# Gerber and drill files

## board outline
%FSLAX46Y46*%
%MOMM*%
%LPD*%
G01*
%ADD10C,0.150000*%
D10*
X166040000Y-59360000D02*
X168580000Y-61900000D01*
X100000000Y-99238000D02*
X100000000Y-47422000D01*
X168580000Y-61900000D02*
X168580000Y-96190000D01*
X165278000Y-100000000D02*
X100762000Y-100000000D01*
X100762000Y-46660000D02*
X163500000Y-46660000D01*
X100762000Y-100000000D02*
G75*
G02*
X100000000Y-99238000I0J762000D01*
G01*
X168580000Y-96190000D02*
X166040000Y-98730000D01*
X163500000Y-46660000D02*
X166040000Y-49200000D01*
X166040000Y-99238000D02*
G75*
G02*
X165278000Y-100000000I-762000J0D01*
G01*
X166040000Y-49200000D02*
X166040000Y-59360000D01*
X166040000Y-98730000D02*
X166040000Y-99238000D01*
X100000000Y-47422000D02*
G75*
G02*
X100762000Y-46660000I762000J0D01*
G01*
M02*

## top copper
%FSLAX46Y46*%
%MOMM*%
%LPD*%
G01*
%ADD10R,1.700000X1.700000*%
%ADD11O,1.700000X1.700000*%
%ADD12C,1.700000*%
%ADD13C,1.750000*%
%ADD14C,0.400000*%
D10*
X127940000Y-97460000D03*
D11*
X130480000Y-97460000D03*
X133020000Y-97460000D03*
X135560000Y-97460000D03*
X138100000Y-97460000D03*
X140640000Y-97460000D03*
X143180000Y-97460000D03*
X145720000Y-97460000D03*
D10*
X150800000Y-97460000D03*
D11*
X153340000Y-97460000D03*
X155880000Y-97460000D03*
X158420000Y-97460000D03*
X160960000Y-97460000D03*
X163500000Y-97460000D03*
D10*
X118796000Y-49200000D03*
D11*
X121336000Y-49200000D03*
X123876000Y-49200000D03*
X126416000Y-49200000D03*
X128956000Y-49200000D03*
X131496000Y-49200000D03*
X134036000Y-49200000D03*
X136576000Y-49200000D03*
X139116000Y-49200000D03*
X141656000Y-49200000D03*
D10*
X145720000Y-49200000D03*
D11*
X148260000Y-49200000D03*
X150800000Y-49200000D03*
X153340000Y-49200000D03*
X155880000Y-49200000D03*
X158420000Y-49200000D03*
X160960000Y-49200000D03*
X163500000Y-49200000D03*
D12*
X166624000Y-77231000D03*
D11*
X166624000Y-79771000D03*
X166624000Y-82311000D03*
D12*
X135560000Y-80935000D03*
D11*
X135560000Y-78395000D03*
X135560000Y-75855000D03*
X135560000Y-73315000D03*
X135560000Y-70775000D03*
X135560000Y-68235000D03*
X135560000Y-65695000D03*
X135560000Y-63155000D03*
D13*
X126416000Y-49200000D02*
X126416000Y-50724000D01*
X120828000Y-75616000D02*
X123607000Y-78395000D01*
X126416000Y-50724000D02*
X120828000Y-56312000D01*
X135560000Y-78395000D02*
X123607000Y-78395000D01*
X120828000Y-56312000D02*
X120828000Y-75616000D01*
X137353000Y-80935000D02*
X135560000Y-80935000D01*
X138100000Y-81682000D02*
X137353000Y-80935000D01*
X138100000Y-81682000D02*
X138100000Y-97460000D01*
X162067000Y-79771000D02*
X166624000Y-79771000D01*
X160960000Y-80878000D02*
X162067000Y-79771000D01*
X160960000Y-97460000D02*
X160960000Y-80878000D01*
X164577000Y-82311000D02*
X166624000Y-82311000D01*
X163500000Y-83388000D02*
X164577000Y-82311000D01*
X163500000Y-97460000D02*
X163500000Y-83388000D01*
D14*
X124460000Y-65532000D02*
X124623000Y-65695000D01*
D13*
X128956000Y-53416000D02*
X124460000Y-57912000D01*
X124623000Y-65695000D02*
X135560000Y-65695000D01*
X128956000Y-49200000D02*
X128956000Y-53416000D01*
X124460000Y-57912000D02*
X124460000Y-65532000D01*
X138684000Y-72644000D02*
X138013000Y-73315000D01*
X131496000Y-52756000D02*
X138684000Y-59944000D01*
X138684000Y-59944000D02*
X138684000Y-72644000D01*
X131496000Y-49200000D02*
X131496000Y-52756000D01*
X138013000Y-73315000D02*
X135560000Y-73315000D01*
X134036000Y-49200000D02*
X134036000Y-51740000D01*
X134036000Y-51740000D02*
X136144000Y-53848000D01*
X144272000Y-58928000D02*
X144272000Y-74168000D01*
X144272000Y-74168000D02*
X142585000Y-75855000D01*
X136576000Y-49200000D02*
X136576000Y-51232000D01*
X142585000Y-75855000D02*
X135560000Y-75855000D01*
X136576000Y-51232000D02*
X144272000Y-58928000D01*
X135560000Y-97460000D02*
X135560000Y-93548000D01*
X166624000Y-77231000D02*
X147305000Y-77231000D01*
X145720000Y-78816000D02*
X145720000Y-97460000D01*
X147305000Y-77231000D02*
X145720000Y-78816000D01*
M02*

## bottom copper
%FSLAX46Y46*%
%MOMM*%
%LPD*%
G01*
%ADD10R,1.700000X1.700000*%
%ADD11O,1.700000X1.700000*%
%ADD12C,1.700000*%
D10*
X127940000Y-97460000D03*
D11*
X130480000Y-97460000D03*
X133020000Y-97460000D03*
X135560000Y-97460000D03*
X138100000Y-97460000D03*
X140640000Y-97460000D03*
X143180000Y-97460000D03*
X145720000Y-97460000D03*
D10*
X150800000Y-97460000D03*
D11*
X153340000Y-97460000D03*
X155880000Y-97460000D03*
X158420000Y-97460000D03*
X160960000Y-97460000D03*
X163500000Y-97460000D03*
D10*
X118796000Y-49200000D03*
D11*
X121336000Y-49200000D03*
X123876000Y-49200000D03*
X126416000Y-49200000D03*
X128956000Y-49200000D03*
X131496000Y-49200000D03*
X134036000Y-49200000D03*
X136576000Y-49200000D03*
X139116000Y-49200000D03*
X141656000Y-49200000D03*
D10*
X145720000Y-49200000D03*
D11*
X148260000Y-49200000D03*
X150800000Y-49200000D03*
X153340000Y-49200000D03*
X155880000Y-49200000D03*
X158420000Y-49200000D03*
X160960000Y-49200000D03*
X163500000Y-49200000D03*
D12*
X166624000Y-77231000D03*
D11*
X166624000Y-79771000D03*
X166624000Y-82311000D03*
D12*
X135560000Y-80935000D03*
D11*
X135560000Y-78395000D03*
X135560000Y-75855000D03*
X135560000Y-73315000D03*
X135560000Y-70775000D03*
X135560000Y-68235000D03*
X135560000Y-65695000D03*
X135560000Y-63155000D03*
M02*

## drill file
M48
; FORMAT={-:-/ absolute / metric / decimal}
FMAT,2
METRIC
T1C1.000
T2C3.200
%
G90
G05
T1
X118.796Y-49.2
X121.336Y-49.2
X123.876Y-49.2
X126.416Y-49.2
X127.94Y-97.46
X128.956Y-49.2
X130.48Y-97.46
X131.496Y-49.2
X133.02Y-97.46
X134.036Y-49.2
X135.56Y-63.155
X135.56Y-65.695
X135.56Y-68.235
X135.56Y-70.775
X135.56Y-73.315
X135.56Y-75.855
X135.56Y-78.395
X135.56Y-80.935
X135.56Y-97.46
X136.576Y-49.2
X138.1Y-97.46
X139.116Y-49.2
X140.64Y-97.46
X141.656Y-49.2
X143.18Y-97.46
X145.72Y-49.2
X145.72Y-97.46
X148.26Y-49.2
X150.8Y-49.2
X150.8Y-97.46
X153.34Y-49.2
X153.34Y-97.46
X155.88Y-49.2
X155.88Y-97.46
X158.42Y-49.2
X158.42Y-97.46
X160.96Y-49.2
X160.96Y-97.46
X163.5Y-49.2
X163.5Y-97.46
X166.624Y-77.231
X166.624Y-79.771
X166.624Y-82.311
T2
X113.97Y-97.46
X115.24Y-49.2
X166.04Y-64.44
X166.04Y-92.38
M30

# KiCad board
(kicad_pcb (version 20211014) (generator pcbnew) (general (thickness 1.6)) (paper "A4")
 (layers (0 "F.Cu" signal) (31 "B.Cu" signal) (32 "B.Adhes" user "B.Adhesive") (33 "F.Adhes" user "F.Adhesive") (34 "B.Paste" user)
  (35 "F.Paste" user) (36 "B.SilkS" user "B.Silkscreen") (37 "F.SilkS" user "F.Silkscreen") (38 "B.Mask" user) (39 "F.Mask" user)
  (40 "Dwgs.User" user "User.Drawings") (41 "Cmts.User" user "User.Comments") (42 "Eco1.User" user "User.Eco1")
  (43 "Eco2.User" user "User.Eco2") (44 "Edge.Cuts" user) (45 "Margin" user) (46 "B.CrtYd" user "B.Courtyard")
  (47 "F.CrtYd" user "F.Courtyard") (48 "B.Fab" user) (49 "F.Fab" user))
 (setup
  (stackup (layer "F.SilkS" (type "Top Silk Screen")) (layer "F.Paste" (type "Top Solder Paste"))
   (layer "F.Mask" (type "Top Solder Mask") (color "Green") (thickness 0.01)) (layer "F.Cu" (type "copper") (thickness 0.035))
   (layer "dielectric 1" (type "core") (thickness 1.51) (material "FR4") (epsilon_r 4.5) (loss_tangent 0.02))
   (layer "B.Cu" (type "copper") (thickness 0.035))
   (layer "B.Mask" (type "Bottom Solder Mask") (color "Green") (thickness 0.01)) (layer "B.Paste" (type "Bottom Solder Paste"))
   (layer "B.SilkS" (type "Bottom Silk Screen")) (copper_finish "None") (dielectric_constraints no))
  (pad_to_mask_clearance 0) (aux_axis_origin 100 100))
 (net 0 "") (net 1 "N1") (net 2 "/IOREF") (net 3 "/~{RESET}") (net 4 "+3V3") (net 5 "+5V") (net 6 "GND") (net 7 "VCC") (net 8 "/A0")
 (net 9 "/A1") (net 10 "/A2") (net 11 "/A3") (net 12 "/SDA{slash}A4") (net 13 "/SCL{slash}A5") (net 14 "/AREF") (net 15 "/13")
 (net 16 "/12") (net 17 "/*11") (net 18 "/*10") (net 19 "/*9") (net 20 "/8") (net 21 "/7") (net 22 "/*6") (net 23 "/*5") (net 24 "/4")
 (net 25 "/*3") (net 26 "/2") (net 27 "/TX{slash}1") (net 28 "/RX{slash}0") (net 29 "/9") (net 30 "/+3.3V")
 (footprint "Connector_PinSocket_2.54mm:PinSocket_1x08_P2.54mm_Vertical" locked (layer "F.Cu") (at 127.94 97.46 90)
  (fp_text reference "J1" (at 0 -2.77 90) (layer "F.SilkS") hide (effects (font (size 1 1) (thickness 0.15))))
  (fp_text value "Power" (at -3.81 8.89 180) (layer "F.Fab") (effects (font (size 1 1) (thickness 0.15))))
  (pad "1" thru_hole rect locked (at 0 0 90) (size 1.7 1.7) (drill 1) (layers *.Cu *.Mask) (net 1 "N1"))
  (pad "2" thru_hole oval locked (at 0 2.54 90) (size 1.7 1.7) (drill 1) (layers *.Cu *.Mask) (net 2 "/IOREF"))
  (pad "3" thru_hole oval locked (at 0 5.08 90) (size 1.7 1.7) (drill 1) (layers *.Cu *.Mask) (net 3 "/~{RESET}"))
  (pad "4" thru_hole oval locked (at 0 7.62 90) (size 1.7 1.7) (drill 1) (layers *.Cu *.Mask) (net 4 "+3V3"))
  (pad "5" thru_hole oval locked (at 0 10.16 90) (size 1.7 1.7) (drill 1) (layers *.Cu *.Mask) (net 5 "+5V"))
  (pad "6" thru_hole oval locked (at 0 12.7 90) (size 1.7 1.7) (drill 1) (layers *.Cu *.Mask) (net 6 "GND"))
  (pad "7" thru_hole oval locked (at 0 15.24 90) (size 1.7 1.7) (drill 1) (layers *.Cu *.Mask) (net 6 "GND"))
  (pad "8" thru_hole oval locked (at 0 17.78 90) (size 1.7 1.7) (drill 1) (layers *.Cu *.Mask) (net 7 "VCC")))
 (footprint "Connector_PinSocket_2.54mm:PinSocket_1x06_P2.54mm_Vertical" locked (layer "F.Cu") (at 150.8 97.46 90)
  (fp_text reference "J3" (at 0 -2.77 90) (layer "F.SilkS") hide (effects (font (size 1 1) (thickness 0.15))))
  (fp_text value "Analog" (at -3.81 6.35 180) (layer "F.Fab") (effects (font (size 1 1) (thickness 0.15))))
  (pad "1" thru_hole rect locked (at 0 0 90) (size 1.7 1.7) (drill 1) (layers *.Cu *.Mask) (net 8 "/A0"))
  (pad "2" thru_hole oval locked (at 0 2.54 90) (size 1.7 1.7) (drill 1) (layers *.Cu *.Mask) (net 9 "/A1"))
  (pad "3" thru_hole oval locked (at 0 5.08 90) (size 1.7 1.7) (drill 1) (layers *.Cu *.Mask) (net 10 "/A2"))
  (pad "4" thru_hole oval locked (at 0 7.62 90) (size 1.7 1.7) (drill 1) (layers *.Cu *.Mask) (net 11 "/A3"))
  (pad "5" thru_hole oval locked (at 0 10.16 90) (size 1.7 1.7) (drill 1) (layers *.Cu *.Mask) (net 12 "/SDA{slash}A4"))
  (pad "6" thru_hole oval locked (at 0 12.7 90) (size 1.7 1.7) (drill 1) (layers *.Cu *.Mask) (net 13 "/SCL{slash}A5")))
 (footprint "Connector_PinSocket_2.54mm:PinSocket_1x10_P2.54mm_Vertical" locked (layer "F.Cu") (at 118.796 49.2 90)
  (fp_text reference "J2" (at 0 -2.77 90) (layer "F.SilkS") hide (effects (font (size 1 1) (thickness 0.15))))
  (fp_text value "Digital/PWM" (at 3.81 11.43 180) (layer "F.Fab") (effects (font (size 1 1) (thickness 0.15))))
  (pad "1" thru_hole rect locked (at 0 0 90) (size 1.7 1.7) (drill 1) (layers *.Cu *.Mask) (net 13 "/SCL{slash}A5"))
  (pad "2" thru_hole oval locked (at 0 2.54 90) (size 1.7 1.7) (drill 1) (layers *.Cu *.Mask) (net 12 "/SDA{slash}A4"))
  (pad "3" thru_hole oval locked (at 0 5.08 90) (size 1.7 1.7) (drill 1) (layers *.Cu *.Mask) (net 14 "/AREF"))
  (pad "4" thru_hole oval locked (at 0 7.62 90) (size 1.7 1.7) (drill 1) (layers *.Cu *.Mask) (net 6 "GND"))
  (pad "5" thru_hole oval locked (at 0 10.16 90) (size 1.7 1.7) (drill 1) (layers *.Cu *.Mask) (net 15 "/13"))
  (pad "6" thru_hole oval locked (at 0 12.7 90) (size 1.7 1.7) (drill 1) (layers *.Cu *.Mask) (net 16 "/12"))
  (pad "7" thru_hole oval locked (at 0 15.24 90) (size 1.7 1.7) (drill 1) (layers *.Cu *.Mask) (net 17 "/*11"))
  (pad "8" thru_hole oval locked (at 0 17.78 90) (size 1.7 1.7) (drill 1) (layers *.Cu *.Mask) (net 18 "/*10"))
  (pad "9" thru_hole oval locked (at 0 20.32 90) (size 1.7 1.7) (drill 1) (layers *.Cu *.Mask) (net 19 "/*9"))
  (pad "10" thru_hole oval locked (at 0 22.86 90) (size 1.7 1.7) (drill 1) (layers *.Cu *.Mask) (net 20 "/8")))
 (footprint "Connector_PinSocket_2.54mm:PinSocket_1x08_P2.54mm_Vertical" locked (layer "F.Cu") (at 145.72 49.2 90)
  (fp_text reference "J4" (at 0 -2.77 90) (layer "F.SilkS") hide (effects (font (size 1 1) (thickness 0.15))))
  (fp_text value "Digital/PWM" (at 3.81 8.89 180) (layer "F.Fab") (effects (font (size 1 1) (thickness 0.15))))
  (pad "1" thru_hole rect locked (at 0 0 90) (size 1.7 1.7) (drill 1) (layers *.Cu *.Mask) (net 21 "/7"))
  (pad "2" thru_hole oval locked (at 0 2.54 90) (size 1.7 1.7) (drill 1) (layers *.Cu *.Mask) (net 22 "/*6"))
  (pad "3" thru_hole oval locked (at 0 5.08 90) (size 1.7 1.7) (drill 1) (layers *.Cu *.Mask) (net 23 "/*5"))
  (pad "4" thru_hole oval locked (at 0 7.62 90) (size 1.7 1.7) (drill 1) (layers *.Cu *.Mask) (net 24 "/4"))
  (pad "5" thru_hole oval locked (at 0 10.16 90) (size 1.7 1.7) (drill 1) (layers *.Cu *.Mask) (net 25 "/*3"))
  (pad "6" thru_hole oval locked (at 0 12.7 90) (size 1.7 1.7) (drill 1) (layers *.Cu *.Mask) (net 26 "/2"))
  (pad "7" thru_hole oval locked (at 0 15.24 90) (size 1.7 1.7) (drill 1) (layers *.Cu *.Mask) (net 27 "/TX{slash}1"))
  (pad "8" thru_hole oval locked (at 0 17.78 90) (size 1.7 1.7) (drill 1) (layers *.Cu *.Mask) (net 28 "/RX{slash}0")))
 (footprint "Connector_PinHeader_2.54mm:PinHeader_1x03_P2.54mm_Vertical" (layer "F.Cu") (at 166.624 77.231)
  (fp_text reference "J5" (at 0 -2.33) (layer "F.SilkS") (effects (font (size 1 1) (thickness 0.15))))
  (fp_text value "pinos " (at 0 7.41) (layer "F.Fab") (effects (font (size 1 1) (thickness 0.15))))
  (pad "1" thru_hole circle (at 0 0) (size 1.7 1.7) (drill 1) (layers *.Cu *.Mask "Dwgs.User") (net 7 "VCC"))
  (pad "2" thru_hole oval (at 0 2.54) (size 1.7 1.7) (drill 1) (layers *.Cu *.Mask) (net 12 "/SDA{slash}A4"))
  (pad "3" thru_hole oval (at 0 5.08) (size 1.7 1.7) (drill 1) (layers *.Cu *.Mask) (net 13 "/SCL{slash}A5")))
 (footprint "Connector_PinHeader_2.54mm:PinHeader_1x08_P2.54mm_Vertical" (layer "F.Cu") (at 135.56 80.935 180)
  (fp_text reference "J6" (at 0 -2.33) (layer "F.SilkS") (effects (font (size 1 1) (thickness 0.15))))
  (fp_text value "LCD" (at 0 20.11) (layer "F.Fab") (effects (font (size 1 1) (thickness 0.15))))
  (pad "1" thru_hole circle (at 0 0 180) (size 1.7 1.7) (drill 1) (layers *.Cu *.Mask) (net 5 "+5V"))
  (pad "2" thru_hole oval (at 0 2.54 180) (size 1.7 1.7) (drill 1) (layers *.Cu *.Mask) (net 6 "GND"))
  (pad "3" thru_hole oval (at 0 5.08 180) (size 1.7 1.7) (drill 1) (layers *.Cu *.Mask) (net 18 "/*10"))
  (pad "4" thru_hole oval (at 0 7.62 180) (size 1.7 1.7) (drill 1) (layers *.Cu *.Mask) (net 16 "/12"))
  (pad "5" thru_hole oval (at 0 10.16 180) (size 1.7 1.7) (drill 1) (layers *.Cu *.Mask) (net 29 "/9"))
  (pad "6" thru_hole oval (at 0 12.7 180) (size 1.7 1.7) (drill 1) (layers *.Cu *.Mask) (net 17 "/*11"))
  (pad "7" thru_hole oval (at 0 15.24 180) (size 1.7 1.7) (drill 1) (layers *.Cu *.Mask) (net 15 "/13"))
  (pad "8" thru_hole oval (at 0 17.78 180) (size 1.7 1.7) (drill 1) (layers *.Cu *.Mask) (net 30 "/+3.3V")))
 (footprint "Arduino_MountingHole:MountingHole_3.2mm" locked (layer "F.Cu") (at 115.24 49.2)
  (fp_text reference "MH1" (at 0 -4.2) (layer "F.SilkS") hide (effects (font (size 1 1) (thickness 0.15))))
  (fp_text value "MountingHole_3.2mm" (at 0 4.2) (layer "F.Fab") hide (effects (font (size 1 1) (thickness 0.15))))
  (pad "" np_thru_hole circle locked (at 0 0) (size 3.2 3.2) (drill 3.2) (layers *.Cu *.Mask)))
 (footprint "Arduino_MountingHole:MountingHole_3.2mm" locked (layer "F.Cu") (at 113.97 97.46)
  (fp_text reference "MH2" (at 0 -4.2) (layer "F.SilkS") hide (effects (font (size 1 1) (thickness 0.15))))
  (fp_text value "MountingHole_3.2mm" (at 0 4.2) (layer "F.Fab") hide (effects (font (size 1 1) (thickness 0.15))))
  (pad "" np_thru_hole circle locked (at 0 0) (size 3.2 3.2) (drill 3.2) (layers *.Cu *.Mask)))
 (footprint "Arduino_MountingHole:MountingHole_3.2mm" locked (layer "F.Cu") (at 166.04 64.44)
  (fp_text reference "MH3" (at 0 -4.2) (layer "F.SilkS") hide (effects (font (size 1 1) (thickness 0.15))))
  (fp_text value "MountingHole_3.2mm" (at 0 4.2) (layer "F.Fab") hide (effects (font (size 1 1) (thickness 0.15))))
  (pad "" np_thru_hole circle locked (at 0 0) (size 3.2 3.2) (drill 3.2) (layers *.Cu *.Mask)))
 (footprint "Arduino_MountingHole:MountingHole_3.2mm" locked (layer "F.Cu") (at 166.04 92.38)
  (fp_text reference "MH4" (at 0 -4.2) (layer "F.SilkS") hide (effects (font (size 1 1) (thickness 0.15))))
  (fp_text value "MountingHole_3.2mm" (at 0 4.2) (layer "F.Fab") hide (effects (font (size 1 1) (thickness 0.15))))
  (pad "" np_thru_hole circle locked (at 0 0) (size 3.2 3.2) (drill 3.2) (layers *.Cu *.Mask)))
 (gr_line (start 166.04 59.36) (end 168.58 61.9) (layer "Edge.Cuts") (width 0.15))
 (gr_line (start 100 99.238) (end 100 47.422) (layer "Edge.Cuts") (width 0.15))
 (gr_line (start 168.58 61.9) (end 168.58 96.19) (layer "Edge.Cuts") (width 0.15))
 (gr_line (start 165.278 100) (end 100.762 100) (layer "Edge.Cuts") (width 0.15))
 (gr_line (start 100.762 46.66) (end 163.5 46.66) (layer "Edge.Cuts") (width 0.15))
 (gr_arc (start 100.762 100) (mid 100.223185 99.776815) (end 100 99.238) (layer "Edge.Cuts") (width 0.15))
 (gr_line (start 168.58 96.19) (end 166.04 98.73) (layer "Edge.Cuts") (width 0.15))
 (gr_line (start 163.5 46.66) (end 166.04 49.2) (layer "Edge.Cuts") (width 0.15))
 (gr_arc (start 166.04 99.238) (mid 165.816815 99.776815) (end 165.278 100) (layer "Edge.Cuts") (width 0.15))
 (gr_line (start 166.04 49.2) (end 166.04 59.36) (layer "Edge.Cuts") (width 0.15))
 (gr_line (start 166.04 98.73) (end 166.04 99.238) (layer "Edge.Cuts") (width 0.15))
 (gr_arc (start 100 47.422) (mid 100.223185 46.883185) (end 100.762 46.66) (layer "Edge.Cuts") (width 0.15))
 (segment (start 126.416 49.2) (end 126.416 50.724) (width 1.75) (layer "F.Cu") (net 6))
 (segment (start 120.828 75.616) (end 123.607 78.395) (width 1.75) (layer "F.Cu") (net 6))
 (segment (start 126.416 50.724) (end 120.828 56.312) (width 1.75) (layer "F.Cu") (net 6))
 (segment (start 135.56 78.395) (end 123.607 78.395) (width 1.75) (layer "F.Cu") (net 6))
 (segment (start 120.828 56.312) (end 120.828 75.616) (width 1.75) (layer "F.Cu") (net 6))
 (segment (start 137.353 80.935) (end 135.56 80.935) (width 1.75) (layer "F.Cu") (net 5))
 (segment (start 138.1 81.682) (end 137.353 80.935) (width 1.75) (layer "F.Cu") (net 5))
 (segment (start 138.1 81.682) (end 138.1 97.46) (width 1.75) (layer "F.Cu") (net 5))
 (segment (start 162.067 79.771) (end 166.624 79.771) (width 1.75) (layer "F.Cu") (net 12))
 (segment (start 160.96 80.878) (end 162.067 79.771) (width 1.75) (layer "F.Cu") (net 12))
 (segment (start 160.96 97.46) (end 160.96 80.878) (width 1.75) (layer "F.Cu") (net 12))
 (segment (start 164.577 82.311) (end 166.624 82.311) (width 1.75) (layer "F.Cu") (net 13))
 (segment (start 163.5 83.388) (end 164.577 82.311) (width 1.75) (layer "F.Cu") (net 13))
 (segment (start 163.5 97.46) (end 163.5 83.388) (width 1.75) (layer "F.Cu") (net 13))
 (segment (start 124.46 65.532) (end 124.623 65.695) (width 0.4) (layer "F.Cu") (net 15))
 (segment (start 128.956 53.416) (end 124.46 57.912) (width 1.75) (layer "F.Cu") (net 15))
 (segment (start 124.623 65.695) (end 135.56 65.695) (width 1.75) (layer "F.Cu") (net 15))
 (segment (start 128.956 49.2) (end 128.956 53.416) (width 1.75) (layer "F.Cu") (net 15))
 (segment (start 124.46 57.912) (end 124.46 65.532) (width 1.75) (layer "F.Cu") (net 15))
 (segment (start 138.684 72.644) (end 138.013 73.315) (width 1.75) (layer "F.Cu") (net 16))
 (segment (start 131.496 52.756) (end 138.684 59.944) (width 1.75) (layer "F.Cu") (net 16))
 (segment (start 138.684 59.944) (end 138.684 72.644) (width 1.75) (layer "F.Cu") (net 16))
 (segment (start 131.496 49.2) (end 131.496 52.756) (width 1.75) (layer "F.Cu") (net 16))
 (segment (start 138.013 73.315) (end 135.56 73.315) (width 1.75) (layer "F.Cu") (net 16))
 (segment (start 134.036 49.2) (end 134.036 51.74) (width 1.75) (layer "F.Cu") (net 17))
 (segment (start 134.036 51.74) (end 136.144 53.848) (width 1.75) (layer "F.Cu") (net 17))
 (segment (start 144.272 58.928) (end 144.272 74.168) (width 1.75) (layer "F.Cu") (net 18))
 (segment (start 144.272 74.168) (end 142.585 75.855) (width 1.75) (layer "F.Cu") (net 18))
 (segment (start 136.576 49.2) (end 136.576 51.232) (width 1.75) (layer "F.Cu") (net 18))
 (segment (start 142.585 75.855) (end 135.56 75.855) (width 1.75) (layer "F.Cu") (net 18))
 (segment (start 136.576 51.232) (end 144.272 58.928) (width 1.75) (layer "F.Cu") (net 18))
 (segment (start 135.56 97.46) (end 135.56 93.548) (width 1.75) (layer "F.Cu") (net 4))
 (segment (start 166.624 77.231) (end 147.305 77.231) (width 1.75) (layer "F.Cu") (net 7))
 (segment (start 145.72 78.816) (end 145.72 97.46) (width 1.75) (layer "F.Cu") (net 7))
 (segment (start 147.305 77.231) (end 145.72 78.816) (width 1.75) (layer "F.Cu") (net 7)))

